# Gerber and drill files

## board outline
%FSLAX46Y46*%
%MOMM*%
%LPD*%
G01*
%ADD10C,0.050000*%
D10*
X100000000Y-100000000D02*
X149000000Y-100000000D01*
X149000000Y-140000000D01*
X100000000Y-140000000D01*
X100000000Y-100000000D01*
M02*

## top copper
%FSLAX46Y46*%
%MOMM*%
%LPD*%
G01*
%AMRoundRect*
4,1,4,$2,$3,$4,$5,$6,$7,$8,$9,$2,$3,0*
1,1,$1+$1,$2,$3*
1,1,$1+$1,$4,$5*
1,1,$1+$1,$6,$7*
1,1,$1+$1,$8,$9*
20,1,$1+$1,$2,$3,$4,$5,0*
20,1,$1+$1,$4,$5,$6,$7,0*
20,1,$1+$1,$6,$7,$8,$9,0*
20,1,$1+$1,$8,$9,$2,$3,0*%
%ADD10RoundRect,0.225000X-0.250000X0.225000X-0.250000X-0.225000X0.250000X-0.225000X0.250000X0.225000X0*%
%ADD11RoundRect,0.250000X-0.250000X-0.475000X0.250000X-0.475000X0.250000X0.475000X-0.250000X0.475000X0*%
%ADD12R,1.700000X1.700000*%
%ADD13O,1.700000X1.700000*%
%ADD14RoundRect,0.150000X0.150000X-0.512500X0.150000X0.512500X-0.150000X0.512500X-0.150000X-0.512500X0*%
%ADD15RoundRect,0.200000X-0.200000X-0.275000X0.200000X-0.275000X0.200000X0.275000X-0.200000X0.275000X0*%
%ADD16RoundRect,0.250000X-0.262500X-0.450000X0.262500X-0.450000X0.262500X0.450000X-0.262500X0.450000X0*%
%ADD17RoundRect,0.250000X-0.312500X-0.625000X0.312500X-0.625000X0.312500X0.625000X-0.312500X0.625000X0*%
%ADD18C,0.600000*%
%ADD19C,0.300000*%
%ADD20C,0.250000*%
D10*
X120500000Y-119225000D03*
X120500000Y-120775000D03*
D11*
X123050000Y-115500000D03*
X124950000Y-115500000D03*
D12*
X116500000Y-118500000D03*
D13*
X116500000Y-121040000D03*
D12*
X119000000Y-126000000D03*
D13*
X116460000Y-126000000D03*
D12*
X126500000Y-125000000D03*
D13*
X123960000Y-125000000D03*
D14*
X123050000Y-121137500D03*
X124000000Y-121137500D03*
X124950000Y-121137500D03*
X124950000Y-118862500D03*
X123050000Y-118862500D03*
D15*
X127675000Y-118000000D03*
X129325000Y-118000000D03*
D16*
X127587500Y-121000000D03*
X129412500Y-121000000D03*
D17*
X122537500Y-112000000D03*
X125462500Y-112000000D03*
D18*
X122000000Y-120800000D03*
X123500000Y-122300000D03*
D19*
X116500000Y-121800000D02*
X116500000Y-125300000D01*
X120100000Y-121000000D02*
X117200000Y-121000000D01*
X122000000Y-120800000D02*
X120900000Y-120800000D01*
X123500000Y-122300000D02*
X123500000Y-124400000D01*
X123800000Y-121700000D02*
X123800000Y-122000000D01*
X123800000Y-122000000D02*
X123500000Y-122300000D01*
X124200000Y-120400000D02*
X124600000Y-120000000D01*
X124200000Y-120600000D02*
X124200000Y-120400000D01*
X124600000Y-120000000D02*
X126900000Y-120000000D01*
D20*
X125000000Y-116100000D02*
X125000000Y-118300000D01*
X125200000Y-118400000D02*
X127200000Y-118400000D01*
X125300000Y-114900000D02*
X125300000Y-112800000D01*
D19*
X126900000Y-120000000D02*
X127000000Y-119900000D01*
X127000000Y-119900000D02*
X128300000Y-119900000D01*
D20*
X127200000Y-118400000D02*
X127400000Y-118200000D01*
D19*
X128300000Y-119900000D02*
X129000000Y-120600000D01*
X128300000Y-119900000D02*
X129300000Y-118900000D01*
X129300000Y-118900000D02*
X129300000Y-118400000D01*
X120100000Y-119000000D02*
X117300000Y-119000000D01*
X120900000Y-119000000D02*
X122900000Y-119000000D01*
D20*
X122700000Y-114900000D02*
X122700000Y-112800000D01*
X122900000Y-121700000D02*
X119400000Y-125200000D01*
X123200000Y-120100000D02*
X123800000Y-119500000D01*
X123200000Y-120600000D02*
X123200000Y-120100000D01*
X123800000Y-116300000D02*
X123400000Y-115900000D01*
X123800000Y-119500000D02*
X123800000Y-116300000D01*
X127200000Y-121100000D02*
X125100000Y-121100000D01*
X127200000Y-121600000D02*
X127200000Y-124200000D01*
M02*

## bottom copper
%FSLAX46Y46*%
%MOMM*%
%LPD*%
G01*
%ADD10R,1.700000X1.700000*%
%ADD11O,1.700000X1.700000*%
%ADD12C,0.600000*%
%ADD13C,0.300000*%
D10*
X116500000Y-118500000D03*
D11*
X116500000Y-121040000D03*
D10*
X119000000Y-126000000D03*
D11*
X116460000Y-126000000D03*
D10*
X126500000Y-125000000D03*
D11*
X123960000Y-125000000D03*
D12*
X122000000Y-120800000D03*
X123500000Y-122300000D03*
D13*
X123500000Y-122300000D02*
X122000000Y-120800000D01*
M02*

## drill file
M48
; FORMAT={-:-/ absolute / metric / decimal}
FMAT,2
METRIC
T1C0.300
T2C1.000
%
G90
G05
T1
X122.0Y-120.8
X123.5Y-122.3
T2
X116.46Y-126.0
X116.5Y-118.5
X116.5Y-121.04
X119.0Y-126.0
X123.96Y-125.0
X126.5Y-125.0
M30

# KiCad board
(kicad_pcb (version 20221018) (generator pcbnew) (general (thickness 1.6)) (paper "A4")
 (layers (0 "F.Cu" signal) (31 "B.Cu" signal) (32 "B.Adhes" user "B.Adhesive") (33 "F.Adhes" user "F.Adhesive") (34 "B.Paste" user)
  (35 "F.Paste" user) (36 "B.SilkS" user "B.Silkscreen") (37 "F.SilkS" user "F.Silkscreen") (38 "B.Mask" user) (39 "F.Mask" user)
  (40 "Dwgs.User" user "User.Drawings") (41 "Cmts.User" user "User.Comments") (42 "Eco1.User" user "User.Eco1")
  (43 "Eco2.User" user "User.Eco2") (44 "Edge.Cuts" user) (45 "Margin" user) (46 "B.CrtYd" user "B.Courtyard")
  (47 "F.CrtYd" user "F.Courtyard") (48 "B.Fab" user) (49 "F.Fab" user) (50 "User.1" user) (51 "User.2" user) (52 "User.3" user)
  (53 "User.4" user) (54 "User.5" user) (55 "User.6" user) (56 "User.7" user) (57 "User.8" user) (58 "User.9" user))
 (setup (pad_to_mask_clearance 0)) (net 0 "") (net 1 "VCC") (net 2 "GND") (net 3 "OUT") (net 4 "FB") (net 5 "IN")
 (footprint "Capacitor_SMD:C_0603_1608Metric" (layer "F.Cu") (at 120.5 120 -90)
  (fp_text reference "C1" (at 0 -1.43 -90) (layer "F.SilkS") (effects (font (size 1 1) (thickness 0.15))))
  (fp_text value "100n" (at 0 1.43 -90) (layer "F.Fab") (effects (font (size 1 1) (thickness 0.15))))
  (pad "1" smd roundrect (at -0.775 0 270) (size 0.9 0.95) (layers "F.Cu" "F.Paste" "F.Mask") (roundrect_rratio 0.25) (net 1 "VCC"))
  (pad "2" smd roundrect (at 0.775 0 270) (size 0.9 0.95) (layers "F.Cu" "F.Paste" "F.Mask") (roundrect_rratio 0.25) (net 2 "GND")))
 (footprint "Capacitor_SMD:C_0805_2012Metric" (layer "F.Cu") (at 124 115.5)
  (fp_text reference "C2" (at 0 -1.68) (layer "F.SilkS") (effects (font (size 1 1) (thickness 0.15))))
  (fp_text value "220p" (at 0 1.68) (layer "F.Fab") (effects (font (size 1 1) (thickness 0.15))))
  (pad "1" smd roundrect (at -0.95 0) (size 1 1.45) (layers "F.Cu" "F.Paste" "F.Mask") (roundrect_rratio 0.25) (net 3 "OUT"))
  (pad "2" smd roundrect (at 0.95 0) (size 1 1.45) (layers "F.Cu" "F.Paste" "F.Mask") (roundrect_rratio 0.25) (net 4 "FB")))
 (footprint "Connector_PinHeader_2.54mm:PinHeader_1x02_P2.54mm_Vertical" (layer "F.Cu") (at 116.5 118.5)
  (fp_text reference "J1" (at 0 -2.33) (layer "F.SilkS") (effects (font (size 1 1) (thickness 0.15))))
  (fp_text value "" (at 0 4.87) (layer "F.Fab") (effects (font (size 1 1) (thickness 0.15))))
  (pad "1" thru_hole rect (at 0 0) (size 1.7 1.7) (drill 1) (layers "*.Cu" "*.Mask") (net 1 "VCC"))
  (pad "2" thru_hole oval (at 0 2.54) (size 1.7 1.7) (drill 1) (layers "*.Cu" "*.Mask") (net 2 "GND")))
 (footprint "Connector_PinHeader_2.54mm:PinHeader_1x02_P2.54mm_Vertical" (layer "F.Cu") (at 119 126 -90)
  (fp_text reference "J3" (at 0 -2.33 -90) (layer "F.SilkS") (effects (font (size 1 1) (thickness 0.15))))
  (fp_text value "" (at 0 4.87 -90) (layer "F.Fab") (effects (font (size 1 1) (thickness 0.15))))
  (pad "1" thru_hole rect (at 0 0 270) (size 1.7 1.7) (drill 1) (layers "*.Cu" "*.Mask") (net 3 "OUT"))
  (pad "2" thru_hole oval (at 0 2.54 270) (size 1.7 1.7) (drill 1) (layers "*.Cu" "*.Mask") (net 2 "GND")))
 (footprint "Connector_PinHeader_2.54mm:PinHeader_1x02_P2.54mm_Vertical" (layer "F.Cu") (at 126.5 125 -90)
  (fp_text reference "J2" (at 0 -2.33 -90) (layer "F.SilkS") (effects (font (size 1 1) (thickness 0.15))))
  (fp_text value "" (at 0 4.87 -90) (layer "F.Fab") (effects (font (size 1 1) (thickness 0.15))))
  (pad "1" thru_hole rect (at 0 0 270) (size 1.7 1.7) (drill 1) (layers "*.Cu" "*.Mask") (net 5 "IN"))
  (pad "2" thru_hole oval (at 0 2.54 270) (size 1.7 1.7) (drill 1) (layers "*.Cu" "*.Mask") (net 2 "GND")))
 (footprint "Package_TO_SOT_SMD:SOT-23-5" (layer "F.Cu") (at 124 120 90)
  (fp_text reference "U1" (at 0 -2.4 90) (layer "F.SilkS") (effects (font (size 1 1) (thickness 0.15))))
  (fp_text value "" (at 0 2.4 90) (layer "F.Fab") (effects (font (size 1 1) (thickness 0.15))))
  (pad "1" smd roundrect (at -1.1375 -0.95 90) (size 1.325 0.6) (layers "F.Cu" "F.Paste" "F.Mask") (roundrect_rratio 0.25) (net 3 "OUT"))
  (pad "2" smd roundrect (at -1.1375 0 90) (size 1.325 0.6) (layers "F.Cu" "F.Paste" "F.Mask") (roundrect_rratio 0.25) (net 2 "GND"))
  (pad "3" smd roundrect (at -1.1375 0.95 90) (size 1.325 0.6) (layers "F.Cu" "F.Paste" "F.Mask") (roundrect_rratio 0.25) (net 5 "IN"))
  (pad "4" smd roundrect (at 1.1375 0.95 90) (size 1.325 0.6) (layers "F.Cu" "F.Paste" "F.Mask") (roundrect_rratio 0.25) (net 4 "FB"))
  (pad "5" smd roundrect (at 1.1375 -0.95 90) (size 1.325 0.6) (layers "F.Cu" "F.Paste" "F.Mask") (roundrect_rratio 0.25) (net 1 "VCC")))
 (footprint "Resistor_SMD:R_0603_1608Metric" (layer "F.Cu") (at 128.5 118)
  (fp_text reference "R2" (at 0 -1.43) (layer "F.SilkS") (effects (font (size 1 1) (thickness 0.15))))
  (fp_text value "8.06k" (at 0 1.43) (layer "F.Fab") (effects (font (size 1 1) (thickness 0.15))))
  (pad "1" smd roundrect (at -0.825 0) (size 0.8 0.95) (layers "F.Cu" "F.Paste" "F.Mask") (roundrect_rratio 0.25) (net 4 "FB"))
  (pad "2" smd roundrect (at 0.825 0) (size 0.8 0.95) (layers "F.Cu" "F.Paste" "F.Mask") (roundrect_rratio 0.25) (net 2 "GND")))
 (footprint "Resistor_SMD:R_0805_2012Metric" (layer "F.Cu") (at 128.5 121)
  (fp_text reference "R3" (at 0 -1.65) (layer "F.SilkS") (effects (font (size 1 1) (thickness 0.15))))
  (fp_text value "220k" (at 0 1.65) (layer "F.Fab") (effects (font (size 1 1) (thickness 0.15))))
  (pad "1" smd roundrect (at -0.9125 0) (size 1.025 1.4) (layers "F.Cu" "F.Paste" "F.Mask") (roundrect_rratio 0.243902) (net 5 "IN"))
  (pad "2" smd roundrect (at 0.9125 0) (size 1.025 1.4) (layers "F.Cu" "F.Paste" "F.Mask") (roundrect_rratio 0.243902) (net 2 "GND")))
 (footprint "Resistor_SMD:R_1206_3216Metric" (layer "F.Cu") (at 124 112)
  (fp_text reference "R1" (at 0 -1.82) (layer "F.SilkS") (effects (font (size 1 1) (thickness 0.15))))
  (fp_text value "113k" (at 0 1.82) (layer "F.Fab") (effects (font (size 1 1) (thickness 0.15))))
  (pad "1" smd roundrect (at -1.4625 0) (size 1.125 1.75) (layers "F.Cu" "F.Paste" "F.Mask") (roundrect_rratio 0.222222) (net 3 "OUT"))
  (pad "2" smd roundrect (at 1.4625 0) (size 1.125 1.75) (layers "F.Cu" "F.Paste" "F.Mask") (roundrect_rratio 0.222222) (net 4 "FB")))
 (gr_rect (start 100 100) (end 149 140) (stroke (width 0.05) (type default)) (fill none) (layer "Edge.Cuts"))
 (segment (start 116.5 121.8) (end 116.5 125.3) (width 0.3) (layer "F.Cu") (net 2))
 (segment (start 120.1 121) (end 117.2 121) (width 0.3) (layer "F.Cu") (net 2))
 (segment (start 122 120.8) (end 120.9 120.8) (width 0.3) (layer "F.Cu") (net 2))
 (segment (start 123.5 122.3) (end 123.5 124.4) (width 0.3) (layer "F.Cu") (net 2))
 (segment (start 123.8 121.7) (end 123.8 122) (width 0.3) (layer "F.Cu") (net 2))
 (segment (start 123.8 122) (end 123.5 122.3) (width 0.3) (layer "F.Cu") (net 2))
 (segment (start 124.2 120.4) (end 124.6 120) (width 0.3) (layer "F.Cu") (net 2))
 (segment (start 124.2 120.6) (end 124.2 120.4) (width 0.3) (layer "F.Cu") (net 2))
 (segment (start 124.6 120) (end 126.9 120) (width 0.3) (layer "F.Cu") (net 2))
 (segment (start 125 116.1) (end 125 118.3) (width 0.25) (layer "F.Cu") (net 4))
 (segment (start 125.2 118.4) (end 127.2 118.4) (width 0.25) (layer "F.Cu") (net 4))
 (segment (start 125.3 114.9) (end 125.3 112.8) (width 0.25) (layer "F.Cu") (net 4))
 (segment (start 126.9 120) (end 127 119.9) (width 0.3) (layer "F.Cu") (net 2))
 (segment (start 127 119.9) (end 128.3 119.9) (width 0.3) (layer "F.Cu") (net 2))
 (segment (start 127.2 118.4) (end 127.4 118.2) (width 0.25) (layer "F.Cu") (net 4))
 (segment (start 128.3 119.9) (end 129 120.6) (width 0.3) (layer "F.Cu") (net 2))
 (segment (start 128.3 119.9) (end 129.3 118.9) (width 0.3) (layer "F.Cu") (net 2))
 (segment (start 129.3 118.9) (end 129.3 118.4) (width 0.3) (layer "F.Cu") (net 2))
 (via (at 122 120.8) (size 0.6) (drill 0.3) (layers "F.Cu" "B.Cu") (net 2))
 (via (at 123.5 122.3) (size 0.6) (drill 0.3) (layers "F.Cu" "B.Cu") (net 2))
 (segment (start 120.1 119) (end 117.3 119) (width 0.3) (layer "F.Cu") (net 1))
 (segment (start 120.9 119) (end 122.9 119) (width 0.3) (layer "F.Cu") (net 1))
 (segment (start 122.7 114.9) (end 122.7 112.8) (width 0.25) (layer "F.Cu") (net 3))
 (segment (start 122.9 121.7) (end 119.4 125.2) (width 0.25) (layer "F.Cu") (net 3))
 (segment (start 123.2 120.1) (end 123.8 119.5) (width 0.25) (layer "F.Cu") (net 3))
 (segment (start 123.2 120.6) (end 123.2 120.1) (width 0.25) (layer "F.Cu") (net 3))
 (segment (start 123.5 122.3) (end 122 120.8) (width 0.3) (layer "B.Cu") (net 2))
 (segment (start 123.8 116.3) (end 123.4 115.9) (width 0.25) (layer "F.Cu") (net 3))
 (segment (start 123.8 119.5) (end 123.8 116.3) (width 0.25) (layer "F.Cu") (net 3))
 (segment (start 127.2 121.1) (end 125.1 121.1) (width 0.25) (layer "F.Cu") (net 5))
 (segment (start 127.2 121.6) (end 127.2 124.2) (width 0.25) (layer "F.Cu") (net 5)))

